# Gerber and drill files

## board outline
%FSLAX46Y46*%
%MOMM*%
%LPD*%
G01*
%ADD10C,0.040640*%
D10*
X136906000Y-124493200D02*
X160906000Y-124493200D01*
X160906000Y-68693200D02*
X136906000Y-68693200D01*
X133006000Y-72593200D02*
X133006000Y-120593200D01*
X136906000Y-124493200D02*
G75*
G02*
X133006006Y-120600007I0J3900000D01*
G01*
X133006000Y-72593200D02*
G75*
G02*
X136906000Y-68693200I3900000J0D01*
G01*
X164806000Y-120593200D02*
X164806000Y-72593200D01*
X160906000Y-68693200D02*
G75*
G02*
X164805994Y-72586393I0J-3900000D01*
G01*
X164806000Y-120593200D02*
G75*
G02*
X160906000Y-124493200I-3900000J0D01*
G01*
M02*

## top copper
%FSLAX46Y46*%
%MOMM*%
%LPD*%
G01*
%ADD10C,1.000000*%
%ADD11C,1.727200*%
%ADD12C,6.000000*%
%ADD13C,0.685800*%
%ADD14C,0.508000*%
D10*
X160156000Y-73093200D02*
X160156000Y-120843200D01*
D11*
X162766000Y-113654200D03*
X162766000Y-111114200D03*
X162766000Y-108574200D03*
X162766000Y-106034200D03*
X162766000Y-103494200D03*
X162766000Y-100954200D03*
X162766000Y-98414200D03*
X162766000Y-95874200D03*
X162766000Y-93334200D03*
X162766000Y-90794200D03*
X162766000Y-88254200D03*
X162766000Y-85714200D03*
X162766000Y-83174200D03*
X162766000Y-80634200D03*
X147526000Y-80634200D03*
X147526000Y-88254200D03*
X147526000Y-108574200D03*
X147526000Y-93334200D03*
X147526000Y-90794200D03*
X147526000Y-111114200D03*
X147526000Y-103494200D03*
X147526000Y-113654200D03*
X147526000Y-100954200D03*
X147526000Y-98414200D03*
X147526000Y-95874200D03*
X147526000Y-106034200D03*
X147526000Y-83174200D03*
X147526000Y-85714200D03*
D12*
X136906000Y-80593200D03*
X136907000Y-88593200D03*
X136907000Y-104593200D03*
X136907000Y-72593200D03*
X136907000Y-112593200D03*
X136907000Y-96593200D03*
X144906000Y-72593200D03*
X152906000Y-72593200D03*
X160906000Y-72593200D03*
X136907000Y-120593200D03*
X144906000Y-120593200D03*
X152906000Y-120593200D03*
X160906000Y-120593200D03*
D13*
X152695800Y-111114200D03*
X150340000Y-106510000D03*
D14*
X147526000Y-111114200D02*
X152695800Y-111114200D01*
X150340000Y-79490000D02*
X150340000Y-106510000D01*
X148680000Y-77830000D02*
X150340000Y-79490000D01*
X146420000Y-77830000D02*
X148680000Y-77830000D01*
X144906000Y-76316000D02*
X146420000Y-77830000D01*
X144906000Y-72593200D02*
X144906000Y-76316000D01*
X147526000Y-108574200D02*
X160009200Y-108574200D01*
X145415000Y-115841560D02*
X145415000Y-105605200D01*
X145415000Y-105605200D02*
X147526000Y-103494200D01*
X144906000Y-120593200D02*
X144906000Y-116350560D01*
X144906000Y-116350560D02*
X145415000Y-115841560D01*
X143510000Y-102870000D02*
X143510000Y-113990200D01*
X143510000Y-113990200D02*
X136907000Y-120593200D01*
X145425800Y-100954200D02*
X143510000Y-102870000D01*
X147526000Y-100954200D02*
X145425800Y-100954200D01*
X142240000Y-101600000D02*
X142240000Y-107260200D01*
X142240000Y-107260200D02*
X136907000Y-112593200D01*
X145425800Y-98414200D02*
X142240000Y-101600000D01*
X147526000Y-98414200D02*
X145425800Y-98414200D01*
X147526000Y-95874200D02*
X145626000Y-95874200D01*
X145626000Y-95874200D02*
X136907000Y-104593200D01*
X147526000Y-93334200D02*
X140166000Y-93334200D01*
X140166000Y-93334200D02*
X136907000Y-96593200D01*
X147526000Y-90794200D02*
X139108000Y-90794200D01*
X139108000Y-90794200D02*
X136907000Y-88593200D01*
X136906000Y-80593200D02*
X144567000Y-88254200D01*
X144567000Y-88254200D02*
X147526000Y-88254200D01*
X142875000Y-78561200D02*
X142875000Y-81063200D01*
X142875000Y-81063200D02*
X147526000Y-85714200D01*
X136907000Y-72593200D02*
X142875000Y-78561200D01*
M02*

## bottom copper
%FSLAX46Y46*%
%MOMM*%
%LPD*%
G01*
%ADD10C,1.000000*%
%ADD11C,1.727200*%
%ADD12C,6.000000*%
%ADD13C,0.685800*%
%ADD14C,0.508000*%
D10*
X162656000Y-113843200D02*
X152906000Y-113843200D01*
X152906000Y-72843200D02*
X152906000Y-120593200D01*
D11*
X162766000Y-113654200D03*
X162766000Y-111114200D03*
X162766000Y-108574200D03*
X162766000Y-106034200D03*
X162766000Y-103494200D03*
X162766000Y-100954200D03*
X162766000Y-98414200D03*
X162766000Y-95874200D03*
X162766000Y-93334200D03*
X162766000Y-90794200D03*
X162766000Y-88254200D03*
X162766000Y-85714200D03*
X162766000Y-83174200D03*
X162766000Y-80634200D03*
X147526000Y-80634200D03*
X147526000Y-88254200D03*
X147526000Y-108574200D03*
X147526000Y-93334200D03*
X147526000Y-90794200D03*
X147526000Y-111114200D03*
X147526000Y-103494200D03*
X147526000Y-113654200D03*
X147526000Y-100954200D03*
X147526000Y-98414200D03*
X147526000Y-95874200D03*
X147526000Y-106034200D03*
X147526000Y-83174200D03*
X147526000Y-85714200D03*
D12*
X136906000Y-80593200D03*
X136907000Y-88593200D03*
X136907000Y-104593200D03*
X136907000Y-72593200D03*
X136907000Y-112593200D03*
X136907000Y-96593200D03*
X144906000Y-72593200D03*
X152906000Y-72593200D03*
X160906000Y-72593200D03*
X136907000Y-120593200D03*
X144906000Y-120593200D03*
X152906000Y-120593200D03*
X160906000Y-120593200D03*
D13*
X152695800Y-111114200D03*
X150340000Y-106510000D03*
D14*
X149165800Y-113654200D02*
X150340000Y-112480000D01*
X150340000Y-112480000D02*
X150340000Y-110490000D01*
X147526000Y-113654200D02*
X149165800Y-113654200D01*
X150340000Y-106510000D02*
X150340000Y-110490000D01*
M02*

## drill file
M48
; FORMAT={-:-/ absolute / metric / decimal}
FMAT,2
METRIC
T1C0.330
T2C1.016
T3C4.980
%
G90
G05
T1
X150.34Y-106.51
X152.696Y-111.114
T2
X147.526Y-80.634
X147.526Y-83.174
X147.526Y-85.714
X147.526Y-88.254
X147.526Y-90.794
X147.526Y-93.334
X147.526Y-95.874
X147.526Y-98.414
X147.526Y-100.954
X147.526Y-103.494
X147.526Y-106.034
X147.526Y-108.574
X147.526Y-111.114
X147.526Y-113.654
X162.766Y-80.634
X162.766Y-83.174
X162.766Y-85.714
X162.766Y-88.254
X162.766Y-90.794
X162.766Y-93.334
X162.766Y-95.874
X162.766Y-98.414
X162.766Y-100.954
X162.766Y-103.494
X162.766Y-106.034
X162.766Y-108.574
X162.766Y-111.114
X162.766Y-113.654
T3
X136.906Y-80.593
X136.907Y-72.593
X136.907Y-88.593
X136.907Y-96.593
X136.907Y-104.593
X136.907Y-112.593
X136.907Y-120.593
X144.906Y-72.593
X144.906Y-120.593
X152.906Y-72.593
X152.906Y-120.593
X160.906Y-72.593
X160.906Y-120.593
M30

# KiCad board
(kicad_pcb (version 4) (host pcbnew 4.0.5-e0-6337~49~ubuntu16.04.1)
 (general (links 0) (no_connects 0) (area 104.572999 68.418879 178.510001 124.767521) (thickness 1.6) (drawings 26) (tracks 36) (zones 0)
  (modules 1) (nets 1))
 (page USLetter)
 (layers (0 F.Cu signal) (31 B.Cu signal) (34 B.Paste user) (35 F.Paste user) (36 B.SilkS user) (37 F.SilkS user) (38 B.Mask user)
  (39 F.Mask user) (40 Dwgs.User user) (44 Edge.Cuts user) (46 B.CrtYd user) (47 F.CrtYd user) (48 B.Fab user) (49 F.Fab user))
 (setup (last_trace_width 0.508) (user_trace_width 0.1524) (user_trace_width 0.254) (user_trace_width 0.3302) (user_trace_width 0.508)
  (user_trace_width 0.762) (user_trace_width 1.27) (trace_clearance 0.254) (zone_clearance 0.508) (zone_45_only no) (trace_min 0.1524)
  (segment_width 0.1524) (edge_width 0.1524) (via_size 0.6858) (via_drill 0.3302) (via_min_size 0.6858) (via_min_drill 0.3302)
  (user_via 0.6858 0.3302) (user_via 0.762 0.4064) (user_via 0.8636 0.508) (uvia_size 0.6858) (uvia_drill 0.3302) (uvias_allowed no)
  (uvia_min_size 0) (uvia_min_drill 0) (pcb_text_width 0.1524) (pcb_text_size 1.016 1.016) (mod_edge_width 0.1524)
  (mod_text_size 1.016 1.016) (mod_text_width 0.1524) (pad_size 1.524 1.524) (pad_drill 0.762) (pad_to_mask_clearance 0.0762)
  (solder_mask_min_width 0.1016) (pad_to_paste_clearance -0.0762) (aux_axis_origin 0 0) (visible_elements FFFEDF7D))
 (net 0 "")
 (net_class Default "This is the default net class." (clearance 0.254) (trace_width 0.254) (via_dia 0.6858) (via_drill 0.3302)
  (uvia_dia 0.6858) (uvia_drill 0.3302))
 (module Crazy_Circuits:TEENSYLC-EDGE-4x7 (layer F.Cu) (at 136.906 72.5932)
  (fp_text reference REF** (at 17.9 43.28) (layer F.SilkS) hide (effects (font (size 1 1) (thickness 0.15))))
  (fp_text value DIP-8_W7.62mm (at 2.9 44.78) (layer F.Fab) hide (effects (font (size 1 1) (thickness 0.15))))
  (fp_line (start 25.75 41.25) (end 16 41.25) (layer B.Cu) (width 1)) (fp_line (start 16 0.25) (end 16 48) (layer B.Cu) (width 1))
  (fp_line (start 0 51.9) (end 24 51.9) (layer Edge.Cuts) (width 0.04064))
  (fp_line (start 24 -3.9) (end 0 -3.9) (layer Edge.Cuts) (width 0.04064))
  (fp_line (start -3.9 0) (end -3.9 48) (layer Edge.Cuts) (width 0.04064))
  (fp_arc (start 0 48) (end 0 51.9) (angle 89.9) (layer Edge.Cuts) (width 0.04064))
  (fp_arc (start 0 0) (end -3.9 0) (angle 90) (layer Edge.Cuts) (width 0.04064))
  (fp_line (start 27.9 48) (end 27.9 0) (layer Edge.Cuts) (width 0.04064))
  (fp_arc (start 24 0) (end 24 -3.9) (angle 89.9) (layer Edge.Cuts) (width 0.04064))
  (fp_arc (start 24 48) (end 27.9 48) (angle 90) (layer Edge.Cuts) (width 0.04064))
  (fp_line (start 23.25 0.5) (end 23.25 48.25) (layer F.Cu) (width 1))
  (pad GND thru_hole circle (at 25.86 41.061 180) (size 1.7272 1.7272) (drill 1.016) (layers *.Cu *.Mask F.SilkS))
  (pad 0 thru_hole circle (at 25.86 38.521 180) (size 1.7272 1.7272) (drill 1.016) (layers *.Cu *.Mask F.SilkS))
  (pad 1 thru_hole circle (at 25.86 35.981 180) (size 1.7272 1.7272) (drill 1.016) (layers *.Cu *.Mask F.SilkS))
  (pad 2 thru_hole circle (at 25.86 33.441 180) (size 1.7272 1.7272) (drill 1.016) (layers *.Cu *.Mask F.SilkS))
  (pad 3 thru_hole circle (at 25.86 30.901 180) (size 1.7272 1.7272) (drill 1.016) (layers *.Cu *.Mask F.SilkS))
  (pad 4 thru_hole circle (at 25.86 28.361 180) (size 1.7272 1.7272) (drill 1.016) (layers *.Cu *.Mask F.SilkS))
  (pad 5 thru_hole circle (at 25.86 25.821 180) (size 1.7272 1.7272) (drill 1.016) (layers *.Cu *.Mask F.SilkS))
  (pad 6 thru_hole circle (at 25.86 23.281 180) (size 1.7272 1.7272) (drill 1.016) (layers *.Cu *.Mask F.SilkS))
  (pad 7 thru_hole circle (at 25.86 20.741 180) (size 1.7272 1.7272) (drill 1.016) (layers *.Cu *.Mask F.SilkS))
  (pad 8 thru_hole circle (at 25.86 18.201 180) (size 1.7272 1.7272) (drill 1.016) (layers *.Cu *.Mask F.SilkS))
  (pad 9 thru_hole circle (at 25.86 15.661 180) (size 1.7272 1.7272) (drill 1.016) (layers *.Cu *.Mask F.SilkS))
  (pad 10 thru_hole circle (at 25.86 13.121 180) (size 1.7272 1.7272) (drill 1.016) (layers *.Cu *.Mask F.SilkS))
  (pad 11 thru_hole circle (at 25.86 10.581 180) (size 1.7272 1.7272) (drill 1.016) (layers *.Cu *.Mask F.SilkS))
  (pad 12 thru_hole circle (at 25.86 8.041 180) (size 1.7272 1.7272) (drill 1.016) (layers *.Cu *.Mask F.SilkS))
  (pad 13 thru_hole circle (at 10.62 8.041 180) (size 1.7272 1.7272) (drill 1.016) (layers *.Cu *.Mask F.SilkS))
  (pad 16 thru_hole circle (at 10.62 15.661 180) (size 1.7272 1.7272) (drill 1.016) (layers *.Cu *.Mask F.SilkS))
  (pad 3.3V thru_hole circle (at 10.62 35.981 180) (size 1.7272 1.7272) (drill 1.016) (layers *.Cu *.Mask F.SilkS))
  (pad 18 thru_hole circle (at 10.62 20.741 180) (size 1.7272 1.7272) (drill 1.016) (layers *.Cu *.Mask F.SilkS))
  (pad 17 thru_hole circle (at 10.62 18.201 180) (size 1.7272 1.7272) (drill 1.016) (layers *.Cu *.Mask F.SilkS))
  (pad G3 thru_hole circle (at 10.62 38.521 180) (size 1.7272 1.7272) (drill 1.016) (layers *.Cu *.Mask F.SilkS))
  (pad 22 thru_hole circle (at 10.62 30.901 180) (size 1.7272 1.7272) (drill 1.016) (layers *.Cu *.Mask F.SilkS))
  (pad VIN thru_hole circle (at 10.62 41.061 180) (size 1.7272 1.7272) (drill 1.016) (layers *.Cu *.Mask F.SilkS))
  (pad 21 thru_hole circle (at 10.62 28.361 180) (size 1.7272 1.7272) (drill 1.016) (layers *.Cu *.Mask F.SilkS))
  (pad 20 thru_hole circle (at 10.62 25.821 180) (size 1.7272 1.7272) (drill 1.016) (layers *.Cu *.Mask F.SilkS))
  (pad 19 thru_hole circle (at 10.62 23.281 180) (size 1.7272 1.7272) (drill 1.016) (layers *.Cu *.Mask F.SilkS))
  (pad 23 thru_hole circle (at 10.62 33.441 180) (size 1.7272 1.7272) (drill 1.016) (layers *.Cu *.Mask F.SilkS))
  (pad 14 thru_hole circle (at 10.62 10.581 180) (size 1.7272 1.7272) (drill 1.016) (layers *.Cu *.Mask F.SilkS))
  (pad 15 thru_hole circle (at 10.62 13.121 180) (size 1.7272 1.7272) (drill 1.016) (layers *.Cu *.Mask F.SilkS))
  (pad 16 thru_hole circle (at 0 8 90) (size 6 6) (drill 4.98) (layers *.Cu *.Mask))
  (pad 17 thru_hole circle (at 0.001 16 90) (size 6 6) (drill 4.98) (layers *.Cu *.Mask))
  (pad 19 thru_hole circle (at 0.001 32 90) (size 6 6) (drill 4.98) (layers *.Cu *.Mask))
  (pad 15 thru_hole circle (at 0.001 0 90) (size 6 6) (drill 4.98) (layers *.Cu *.Mask))
  (pad 20 thru_hole circle (at 0.001 40 90) (size 6 6) (drill 4.98) (layers *.Cu *.Mask))
  (pad 18 thru_hole circle (at 0.001 24 90) (size 6 6) (drill 4.98) (layers *.Cu *.Mask))
  (pad VIN thru_hole circle (at 8 0 90) (size 6 6) (drill 4.98) (layers *.Cu *.Mask))
  (pad GND thru_hole circle (at 16 0 90) (size 6 6) (drill 4.98) (layers *.Cu *.Mask))
  (pad 3.3V thru_hole circle (at 24 0 90) (size 6 6) (drill 4.98) (layers *.Cu *.Mask))
  (pad 21 thru_hole circle (at 0.001 48 90) (size 6 6) (drill 4.98) (layers *.Cu *.Mask))
  (pad 22 thru_hole circle (at 8 48 90) (size 6 6) (drill 4.98) (layers *.Cu *.Mask))
  (pad GND thru_hole circle (at 16 48 90) (size 6 6) (drill 4.98) (layers *.Cu *.Mask))
  (pad 3.3V thru_hole circle (at 24 48 90) (size 6 6) (drill 4.98) (layers *.Cu *.Mask)))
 (via (at 152.6958 111.1142) (size 0.6858) (drill 0.3302) (layers F.Cu B.Cu) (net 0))
 (segment (start 147.526 111.1142) (end 152.6958 111.1142) (width 0.508) (layer F.Cu) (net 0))
 (segment (start 149.1658 113.6542) (end 150.34 112.48) (width 0.508) (layer B.Cu) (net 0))
 (segment (start 150.34 112.48) (end 150.34 110.49) (width 0.508) (layer B.Cu) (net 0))
 (segment (start 147.526 113.6542) (end 149.1658 113.6542) (width 0.508) (layer B.Cu) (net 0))
 (segment (start 150.34 106.51) (end 150.34 110.49) (width 0.508) (layer B.Cu) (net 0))
 (segment (start 150.34 79.49) (end 150.34 106.51) (width 0.508) (layer F.Cu) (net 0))
 (via (at 150.34 106.51) (size 0.6858) (drill 0.3302) (layers F.Cu B.Cu) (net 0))
 (segment (start 148.68 77.83) (end 150.34 79.49) (width 0.508) (layer F.Cu) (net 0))
 (segment (start 146.42 77.83) (end 148.68 77.83) (width 0.508) (layer F.Cu) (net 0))
 (segment (start 144.906 76.316) (end 146.42 77.83) (width 0.508) (layer F.Cu) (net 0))
 (segment (start 144.906 72.5932) (end 144.906 76.316) (width 0.508) (layer F.Cu) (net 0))
 (segment (start 147.526 108.5742) (end 160.0092 108.5742) (width 0.508) (layer F.Cu) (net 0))
 (segment (start 145.415 115.84156) (end 145.415 105.6052) (width 0.508) (layer F.Cu) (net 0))
 (segment (start 145.415 105.6052) (end 147.526 103.4942) (width 0.508) (layer F.Cu) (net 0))
 (segment (start 144.906 120.5932) (end 144.906 116.35056) (width 0.508) (layer F.Cu) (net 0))
 (segment (start 144.906 116.35056) (end 145.415 115.84156) (width 0.508) (layer F.Cu) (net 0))
 (segment (start 143.51 102.87) (end 143.51 113.9902) (width 0.508) (layer F.Cu) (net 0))
 (segment (start 143.51 113.9902) (end 136.907 120.5932) (width 0.508) (layer F.Cu) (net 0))
 (segment (start 145.4258 100.9542) (end 143.51 102.87) (width 0.508) (layer F.Cu) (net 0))
 (segment (start 147.526 100.9542) (end 145.4258 100.9542) (width 0.508) (layer F.Cu) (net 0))
 (segment (start 142.24 101.6) (end 142.24 107.2602) (width 0.508) (layer F.Cu) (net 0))
 (segment (start 142.24 107.2602) (end 136.907 112.5932) (width 0.508) (layer F.Cu) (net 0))
 (segment (start 145.4258 98.4142) (end 142.24 101.6) (width 0.508) (layer F.Cu) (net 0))
 (segment (start 147.526 98.4142) (end 145.4258 98.4142) (width 0.508) (layer F.Cu) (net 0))
 (segment (start 147.526 95.8742) (end 145.626 95.8742) (width 0.508) (layer F.Cu) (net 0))
 (segment (start 145.626 95.8742) (end 136.907 104.5932) (width 0.508) (layer F.Cu) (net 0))
 (segment (start 147.526 93.3342) (end 140.166 93.3342) (width 0.508) (layer F.Cu) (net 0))
 (segment (start 140.166 93.3342) (end 136.907 96.5932) (width 0.508) (layer F.Cu) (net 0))
 (segment (start 147.526 90.7942) (end 139.108 90.7942) (width 0.508) (layer F.Cu) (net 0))
 (segment (start 139.108 90.7942) (end 136.907 88.5932) (width 0.508) (layer F.Cu) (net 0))
 (segment (start 136.906 80.5932) (end 144.567 88.2542) (width 0.508) (layer F.Cu) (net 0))
 (segment (start 144.567 88.2542) (end 147.526 88.2542) (width 0.508) (layer F.Cu) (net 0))
 (segment (start 142.875 78.5612) (end 142.875 81.0632) (width 0.508) (layer F.Cu) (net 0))
 (segment (start 142.875 81.0632) (end 147.526 85.7142) (width 0.508) (layer F.Cu) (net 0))
 (segment (start 136.907 72.5932) (end 142.875 78.5612) (width 0.508) (layer F.Cu) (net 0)))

